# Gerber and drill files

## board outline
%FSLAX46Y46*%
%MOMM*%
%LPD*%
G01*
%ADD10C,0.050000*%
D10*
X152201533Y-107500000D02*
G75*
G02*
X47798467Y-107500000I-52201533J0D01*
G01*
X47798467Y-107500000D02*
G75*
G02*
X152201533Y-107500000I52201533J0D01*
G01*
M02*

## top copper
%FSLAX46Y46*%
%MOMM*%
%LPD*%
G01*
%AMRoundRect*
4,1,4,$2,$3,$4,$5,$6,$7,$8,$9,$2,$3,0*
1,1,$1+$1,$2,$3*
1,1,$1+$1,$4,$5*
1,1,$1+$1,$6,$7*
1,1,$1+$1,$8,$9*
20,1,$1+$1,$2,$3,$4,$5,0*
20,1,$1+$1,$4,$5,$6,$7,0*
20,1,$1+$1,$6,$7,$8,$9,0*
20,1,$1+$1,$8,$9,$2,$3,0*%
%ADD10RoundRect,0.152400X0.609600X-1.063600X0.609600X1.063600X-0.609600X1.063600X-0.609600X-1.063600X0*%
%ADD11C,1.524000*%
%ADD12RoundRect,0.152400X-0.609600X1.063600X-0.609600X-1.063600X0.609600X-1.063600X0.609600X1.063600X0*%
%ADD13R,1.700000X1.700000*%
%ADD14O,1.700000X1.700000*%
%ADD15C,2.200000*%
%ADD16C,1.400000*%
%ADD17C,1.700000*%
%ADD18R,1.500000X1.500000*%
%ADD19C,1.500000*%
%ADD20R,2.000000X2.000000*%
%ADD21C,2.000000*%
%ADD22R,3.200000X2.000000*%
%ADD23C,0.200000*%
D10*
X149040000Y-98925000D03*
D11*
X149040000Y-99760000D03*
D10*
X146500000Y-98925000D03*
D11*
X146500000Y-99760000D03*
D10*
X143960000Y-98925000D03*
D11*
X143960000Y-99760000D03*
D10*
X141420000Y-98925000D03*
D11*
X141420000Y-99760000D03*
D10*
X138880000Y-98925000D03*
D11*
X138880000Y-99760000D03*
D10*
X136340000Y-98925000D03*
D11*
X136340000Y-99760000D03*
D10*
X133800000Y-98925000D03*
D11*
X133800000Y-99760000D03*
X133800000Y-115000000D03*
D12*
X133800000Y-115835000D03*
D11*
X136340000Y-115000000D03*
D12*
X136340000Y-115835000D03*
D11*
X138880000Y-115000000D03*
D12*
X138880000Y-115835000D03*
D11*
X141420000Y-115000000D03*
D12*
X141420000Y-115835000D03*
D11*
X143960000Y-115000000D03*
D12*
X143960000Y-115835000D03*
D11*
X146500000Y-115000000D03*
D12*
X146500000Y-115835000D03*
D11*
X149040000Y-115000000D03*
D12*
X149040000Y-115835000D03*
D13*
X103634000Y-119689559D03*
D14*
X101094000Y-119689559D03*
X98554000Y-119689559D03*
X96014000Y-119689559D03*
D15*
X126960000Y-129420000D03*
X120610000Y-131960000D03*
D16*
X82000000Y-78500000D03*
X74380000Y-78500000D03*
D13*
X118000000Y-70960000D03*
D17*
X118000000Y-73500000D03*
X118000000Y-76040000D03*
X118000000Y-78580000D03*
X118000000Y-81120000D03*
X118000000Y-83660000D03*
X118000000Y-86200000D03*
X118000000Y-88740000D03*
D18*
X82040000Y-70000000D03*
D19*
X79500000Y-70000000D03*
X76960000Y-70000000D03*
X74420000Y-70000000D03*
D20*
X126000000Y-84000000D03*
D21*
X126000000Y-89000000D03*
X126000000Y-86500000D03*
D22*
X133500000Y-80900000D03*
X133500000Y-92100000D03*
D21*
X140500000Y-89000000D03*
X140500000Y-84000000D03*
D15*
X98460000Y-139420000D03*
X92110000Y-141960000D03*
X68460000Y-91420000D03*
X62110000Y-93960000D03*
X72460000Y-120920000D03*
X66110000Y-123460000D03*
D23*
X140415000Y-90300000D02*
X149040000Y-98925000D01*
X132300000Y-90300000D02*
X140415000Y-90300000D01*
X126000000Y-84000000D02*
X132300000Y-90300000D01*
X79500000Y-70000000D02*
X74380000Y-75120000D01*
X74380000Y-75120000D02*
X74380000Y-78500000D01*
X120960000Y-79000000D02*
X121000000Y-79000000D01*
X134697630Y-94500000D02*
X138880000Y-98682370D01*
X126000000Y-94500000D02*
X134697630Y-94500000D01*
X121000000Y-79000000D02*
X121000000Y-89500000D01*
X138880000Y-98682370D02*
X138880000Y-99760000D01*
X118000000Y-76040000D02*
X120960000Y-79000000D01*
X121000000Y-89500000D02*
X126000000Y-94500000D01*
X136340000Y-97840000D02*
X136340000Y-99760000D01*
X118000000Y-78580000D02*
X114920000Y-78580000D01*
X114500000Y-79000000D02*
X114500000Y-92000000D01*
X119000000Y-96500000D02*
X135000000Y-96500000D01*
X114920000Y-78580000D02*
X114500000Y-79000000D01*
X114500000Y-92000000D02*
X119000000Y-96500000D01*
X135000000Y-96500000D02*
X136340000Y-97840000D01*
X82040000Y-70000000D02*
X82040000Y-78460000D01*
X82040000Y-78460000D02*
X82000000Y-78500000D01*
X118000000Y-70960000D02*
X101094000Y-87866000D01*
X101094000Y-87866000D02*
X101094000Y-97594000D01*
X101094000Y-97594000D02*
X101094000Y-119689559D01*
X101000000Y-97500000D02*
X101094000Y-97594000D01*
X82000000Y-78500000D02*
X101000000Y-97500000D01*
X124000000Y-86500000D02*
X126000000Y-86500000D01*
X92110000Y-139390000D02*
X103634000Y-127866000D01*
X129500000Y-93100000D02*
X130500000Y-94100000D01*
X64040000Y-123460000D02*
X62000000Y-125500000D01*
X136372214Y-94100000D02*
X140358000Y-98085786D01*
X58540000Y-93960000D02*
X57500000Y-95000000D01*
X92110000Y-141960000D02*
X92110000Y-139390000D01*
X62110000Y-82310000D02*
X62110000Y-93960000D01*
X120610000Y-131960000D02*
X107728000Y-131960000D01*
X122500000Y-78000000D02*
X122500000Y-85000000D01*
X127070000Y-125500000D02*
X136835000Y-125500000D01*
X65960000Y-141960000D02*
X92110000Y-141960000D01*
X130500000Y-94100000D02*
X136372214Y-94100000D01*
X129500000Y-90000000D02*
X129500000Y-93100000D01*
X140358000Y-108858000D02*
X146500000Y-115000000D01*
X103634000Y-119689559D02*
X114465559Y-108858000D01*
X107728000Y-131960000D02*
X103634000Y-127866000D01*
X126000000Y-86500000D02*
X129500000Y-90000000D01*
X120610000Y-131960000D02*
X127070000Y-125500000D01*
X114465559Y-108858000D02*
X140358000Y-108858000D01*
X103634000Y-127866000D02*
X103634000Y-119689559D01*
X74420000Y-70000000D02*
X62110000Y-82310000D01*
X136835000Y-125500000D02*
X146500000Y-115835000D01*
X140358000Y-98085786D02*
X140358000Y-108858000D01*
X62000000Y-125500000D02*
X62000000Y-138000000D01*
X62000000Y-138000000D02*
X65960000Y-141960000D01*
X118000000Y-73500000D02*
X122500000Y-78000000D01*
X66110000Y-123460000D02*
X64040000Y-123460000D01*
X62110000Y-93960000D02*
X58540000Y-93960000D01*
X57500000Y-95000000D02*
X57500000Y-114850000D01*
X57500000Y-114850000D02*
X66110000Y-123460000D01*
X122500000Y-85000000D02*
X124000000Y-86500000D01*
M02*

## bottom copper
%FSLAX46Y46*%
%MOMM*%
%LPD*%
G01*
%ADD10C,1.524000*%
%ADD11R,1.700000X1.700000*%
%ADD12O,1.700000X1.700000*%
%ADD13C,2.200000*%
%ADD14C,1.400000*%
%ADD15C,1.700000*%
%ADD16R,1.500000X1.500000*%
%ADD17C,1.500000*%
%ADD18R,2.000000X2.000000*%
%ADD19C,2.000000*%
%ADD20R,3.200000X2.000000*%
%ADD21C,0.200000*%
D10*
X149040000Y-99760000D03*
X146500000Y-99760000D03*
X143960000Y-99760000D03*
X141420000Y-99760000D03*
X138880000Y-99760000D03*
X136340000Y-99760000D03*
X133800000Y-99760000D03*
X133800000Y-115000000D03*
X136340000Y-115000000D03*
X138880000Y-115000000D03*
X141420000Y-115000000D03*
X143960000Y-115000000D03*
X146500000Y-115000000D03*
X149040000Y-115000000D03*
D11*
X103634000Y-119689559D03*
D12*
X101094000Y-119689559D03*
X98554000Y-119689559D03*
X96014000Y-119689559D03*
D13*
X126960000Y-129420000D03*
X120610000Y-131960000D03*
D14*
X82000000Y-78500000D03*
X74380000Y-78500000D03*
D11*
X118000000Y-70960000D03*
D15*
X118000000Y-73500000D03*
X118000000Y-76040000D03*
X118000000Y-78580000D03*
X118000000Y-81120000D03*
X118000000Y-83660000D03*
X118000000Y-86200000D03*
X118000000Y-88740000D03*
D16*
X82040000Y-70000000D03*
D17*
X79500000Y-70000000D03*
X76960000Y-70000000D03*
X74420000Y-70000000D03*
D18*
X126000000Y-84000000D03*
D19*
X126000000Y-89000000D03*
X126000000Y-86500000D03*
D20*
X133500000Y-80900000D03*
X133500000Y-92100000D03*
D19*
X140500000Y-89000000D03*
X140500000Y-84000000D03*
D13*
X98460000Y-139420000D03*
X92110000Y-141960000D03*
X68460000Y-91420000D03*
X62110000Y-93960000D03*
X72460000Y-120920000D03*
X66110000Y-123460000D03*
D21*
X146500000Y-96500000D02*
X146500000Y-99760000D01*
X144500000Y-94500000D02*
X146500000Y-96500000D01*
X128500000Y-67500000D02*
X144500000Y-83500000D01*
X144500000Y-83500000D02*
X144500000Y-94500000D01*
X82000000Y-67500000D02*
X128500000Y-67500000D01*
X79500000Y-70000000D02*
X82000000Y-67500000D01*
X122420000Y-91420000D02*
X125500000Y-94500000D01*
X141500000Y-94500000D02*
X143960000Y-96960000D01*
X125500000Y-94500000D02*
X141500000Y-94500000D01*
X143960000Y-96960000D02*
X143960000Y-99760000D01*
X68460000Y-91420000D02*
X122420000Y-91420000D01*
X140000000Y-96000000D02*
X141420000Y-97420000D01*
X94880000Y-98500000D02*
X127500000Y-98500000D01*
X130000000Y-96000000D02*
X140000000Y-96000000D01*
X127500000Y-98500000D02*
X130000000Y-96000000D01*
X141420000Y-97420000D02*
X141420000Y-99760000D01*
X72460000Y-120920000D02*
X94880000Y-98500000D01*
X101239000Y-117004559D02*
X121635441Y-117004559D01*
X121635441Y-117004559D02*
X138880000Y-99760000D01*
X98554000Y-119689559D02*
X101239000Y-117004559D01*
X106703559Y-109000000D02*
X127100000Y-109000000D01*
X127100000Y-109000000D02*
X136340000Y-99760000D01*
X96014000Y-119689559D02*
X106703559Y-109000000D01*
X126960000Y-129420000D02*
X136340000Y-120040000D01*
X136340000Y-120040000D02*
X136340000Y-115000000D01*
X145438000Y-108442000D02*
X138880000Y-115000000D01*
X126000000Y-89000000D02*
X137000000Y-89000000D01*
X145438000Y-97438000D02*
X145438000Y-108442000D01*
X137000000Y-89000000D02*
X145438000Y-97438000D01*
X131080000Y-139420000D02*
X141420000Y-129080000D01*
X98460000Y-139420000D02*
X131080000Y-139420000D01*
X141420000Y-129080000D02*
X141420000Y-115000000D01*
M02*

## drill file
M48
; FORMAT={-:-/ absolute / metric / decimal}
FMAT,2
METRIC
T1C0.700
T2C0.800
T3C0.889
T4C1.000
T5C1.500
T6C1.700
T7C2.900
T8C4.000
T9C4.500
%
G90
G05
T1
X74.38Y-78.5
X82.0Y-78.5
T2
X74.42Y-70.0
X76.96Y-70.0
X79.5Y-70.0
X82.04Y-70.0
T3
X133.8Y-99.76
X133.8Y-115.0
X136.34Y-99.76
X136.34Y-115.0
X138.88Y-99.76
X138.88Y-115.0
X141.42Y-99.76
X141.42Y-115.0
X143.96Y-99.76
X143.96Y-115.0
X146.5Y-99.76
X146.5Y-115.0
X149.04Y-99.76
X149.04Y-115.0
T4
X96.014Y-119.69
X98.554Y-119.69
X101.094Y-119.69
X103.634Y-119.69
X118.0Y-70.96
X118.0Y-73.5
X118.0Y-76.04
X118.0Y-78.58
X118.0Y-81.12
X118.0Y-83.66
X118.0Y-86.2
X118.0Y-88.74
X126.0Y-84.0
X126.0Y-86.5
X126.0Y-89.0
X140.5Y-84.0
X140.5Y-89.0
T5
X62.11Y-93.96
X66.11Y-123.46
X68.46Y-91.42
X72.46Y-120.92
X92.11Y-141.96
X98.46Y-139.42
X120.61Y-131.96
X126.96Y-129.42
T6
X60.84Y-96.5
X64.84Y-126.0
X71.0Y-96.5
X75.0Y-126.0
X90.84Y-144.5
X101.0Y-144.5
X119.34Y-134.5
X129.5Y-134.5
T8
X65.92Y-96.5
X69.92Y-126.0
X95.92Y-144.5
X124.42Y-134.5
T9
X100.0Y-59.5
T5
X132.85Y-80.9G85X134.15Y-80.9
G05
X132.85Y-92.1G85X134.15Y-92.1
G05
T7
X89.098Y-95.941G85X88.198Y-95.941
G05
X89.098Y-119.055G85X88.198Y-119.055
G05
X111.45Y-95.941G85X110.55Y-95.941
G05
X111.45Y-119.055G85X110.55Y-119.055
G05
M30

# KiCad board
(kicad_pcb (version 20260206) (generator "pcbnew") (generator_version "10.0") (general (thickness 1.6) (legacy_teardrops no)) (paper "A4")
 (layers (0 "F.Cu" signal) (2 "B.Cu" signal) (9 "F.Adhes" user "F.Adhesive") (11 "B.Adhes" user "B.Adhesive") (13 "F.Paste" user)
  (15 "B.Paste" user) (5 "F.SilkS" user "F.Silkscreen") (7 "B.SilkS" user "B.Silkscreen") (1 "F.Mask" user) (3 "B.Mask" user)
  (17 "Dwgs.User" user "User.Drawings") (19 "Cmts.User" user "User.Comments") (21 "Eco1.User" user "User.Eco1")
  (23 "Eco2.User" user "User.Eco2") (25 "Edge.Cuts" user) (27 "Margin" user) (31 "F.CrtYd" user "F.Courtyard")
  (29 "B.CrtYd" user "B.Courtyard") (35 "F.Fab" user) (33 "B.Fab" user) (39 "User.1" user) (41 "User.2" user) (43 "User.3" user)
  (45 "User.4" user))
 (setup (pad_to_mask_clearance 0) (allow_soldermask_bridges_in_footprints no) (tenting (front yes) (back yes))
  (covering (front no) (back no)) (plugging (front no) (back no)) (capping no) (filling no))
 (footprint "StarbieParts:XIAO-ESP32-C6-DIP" (layer "F.Cu") (at 141.42 107.38)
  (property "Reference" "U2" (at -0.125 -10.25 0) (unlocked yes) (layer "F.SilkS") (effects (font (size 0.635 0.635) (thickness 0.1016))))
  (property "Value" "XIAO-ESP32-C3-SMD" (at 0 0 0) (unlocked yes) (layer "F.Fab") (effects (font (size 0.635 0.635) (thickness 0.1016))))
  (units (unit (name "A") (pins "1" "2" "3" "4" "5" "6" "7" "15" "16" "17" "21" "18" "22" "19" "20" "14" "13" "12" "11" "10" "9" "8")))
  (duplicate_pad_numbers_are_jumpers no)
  (pad "1" smd roundrect (at 7.62 -8.455 90) (size 2.432 1.524) (layers "F.Cu" "F.Mask") (roundrect_rratio 0.1) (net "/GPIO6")
   (thermal_bridge_angle 45))
  (pad "1" thru_hole circle (at 7.62 -7.62 90) (size 1.524 1.524) (drill 0.889) (layers "*.Cu" "*.Mask") (remove_unused_layers no)
   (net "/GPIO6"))
  (pad "2" smd roundrect (at 5.08 -8.455 90) (size 2.432 1.524) (layers "F.Cu" "F.Mask") (roundrect_rratio 0.1) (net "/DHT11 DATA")
   (thermal_bridge_angle 45))
  (pad "2" thru_hole circle (at 5.08 -7.62 90) (size 1.524 1.524) (drill 0.889) (layers "*.Cu" "*.Mask") (remove_unused_layers no)
   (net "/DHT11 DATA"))
  (pad "3" smd roundrect (at 2.54 -8.455 90) (size 2.432 1.524) (layers "F.Cu" "F.Mask") (roundrect_rratio 0.1) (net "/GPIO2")
   (thermal_bridge_angle 45))
  (pad "3" thru_hole circle (at 2.54 -7.62 90) (size 1.524 1.524) (drill 0.889) (layers "*.Cu" "*.Mask") (remove_unused_layers no)
   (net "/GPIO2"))
  (pad "4" smd roundrect (at 0 -8.455 90) (size 2.432 1.524) (layers "F.Cu" "F.Mask") (roundrect_rratio 0.1) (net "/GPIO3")
   (thermal_bridge_angle 45))
  (pad "4" thru_hole circle (at 0 -7.62 90) (size 1.524 1.524) (drill 0.889) (layers "*.Cu" "*.Mask") (remove_unused_layers no)
   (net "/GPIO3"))
  (pad "5" smd roundrect (at -2.54 -8.455 90) (size 2.432 1.524) (layers "F.Cu" "F.Mask") (roundrect_rratio 0.1) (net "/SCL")
   (thermal_bridge_angle 45))
  (pad "5" thru_hole circle (at -2.54 -7.62 90) (size 1.524 1.524) (drill 0.889) (layers "*.Cu" "*.Mask") (remove_unused_layers no)
   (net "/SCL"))
  (pad "6" smd roundrect (at -5.08 -8.455 90) (size 2.432 1.524) (layers "F.Cu" "F.Mask") (roundrect_rratio 0.1) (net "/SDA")
   (thermal_bridge_angle 45))
  (pad "6" thru_hole circle (at -5.08 -7.62 90) (size 1.524 1.524) (drill 0.889) (layers "*.Cu" "*.Mask") (remove_unused_layers no)
   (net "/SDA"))
  (pad "7" smd roundrect (at -7.62 -8.455 90) (size 2.432 1.524) (layers "F.Cu" "F.Mask") (roundrect_rratio 0.1)
   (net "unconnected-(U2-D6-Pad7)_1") (thermal_bridge_angle 45))
  (pad "7" thru_hole circle (at -7.62 -7.62 90) (size 1.524 1.524) (drill 0.889) (layers "*.Cu" "*.Mask") (remove_unused_layers no)
   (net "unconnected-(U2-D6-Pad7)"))
  (pad "8" thru_hole circle (at -7.62 7.62 270) (size 1.524 1.524) (drill 0.889) (layers "*.Cu" "*.Mask") (remove_unused_layers no)
   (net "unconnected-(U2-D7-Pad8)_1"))
  (pad "8" smd roundrect (at -7.62 8.455 270) (size 2.432 1.524) (layers "F.Cu" "F.Mask") (roundrect_rratio 0.1)
   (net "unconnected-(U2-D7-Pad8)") (thermal_bridge_angle 45))
  (pad "9" thru_hole circle (at -5.08 7.62 270) (size 1.524 1.524) (drill 0.889) (layers "*.Cu" "*.Mask") (remove_unused_layers no)
   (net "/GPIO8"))
  (pad "9" smd roundrect (at -5.08 8.455 270) (size 2.432 1.524) (layers "F.Cu" "F.Mask") (roundrect_rratio 0.1) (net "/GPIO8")
   (thermal_bridge_angle 45))
  (pad "10" thru_hole circle (at -2.54 7.62 270) (size 1.524 1.524) (drill 0.889) (layers "*.Cu" "*.Mask") (remove_unused_layers no)
   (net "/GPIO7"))
  (pad "10" smd roundrect (at -2.54 8.455 270) (size 2.432 1.524) (layers "F.Cu" "F.Mask") (roundrect_rratio 0.1) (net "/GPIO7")
   (thermal_bridge_angle 45))
  (pad "11" thru_hole circle (at 0 7.62 270) (size 1.524 1.524) (drill 0.889) (layers "*.Cu" "*.Mask") (remove_unused_layers no)
   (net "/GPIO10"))
  (pad "11" smd roundrect (at 0 8.455 270) (size 2.432 1.524) (layers "F.Cu" "F.Mask") (roundrect_rratio 0.1) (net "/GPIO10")
   (thermal_bridge_angle 45))
  (pad "12" thru_hole circle (at 2.54 7.62 270) (size 1.524 1.524) (drill 0.889) (layers "*.Cu" "*.Mask") (remove_unused_layers no)
   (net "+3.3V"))
  (pad "12" smd roundrect (at 2.54 8.455 270) (size 2.432 1.524) (layers "F.Cu" "F.Mask") (roundrect_rratio 0.1) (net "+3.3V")
   (thermal_bridge_angle 45))
  (pad "13" thru_hole circle (at 5.08 7.62 270) (size 1.524 1.524) (drill 0.889) (layers "*.Cu" "*.Mask") (remove_unused_layers no)
   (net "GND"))
  (pad "13" smd roundrect (at 5.08 8.455 270) (size 2.432 1.524) (layers "F.Cu" "F.Mask") (roundrect_rratio 0.1) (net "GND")
   (thermal_bridge_angle 45))
  (pad "14" thru_hole circle (at 7.62 7.62 270) (size 1.524 1.524) (drill 0.889) (layers "*.Cu" "*.Mask") (remove_unused_layers no)
   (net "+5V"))
  (pad "14" smd roundrect (at 7.62 8.455 270) (size 2.432 1.524) (layers "F.Cu" "F.Mask") (roundrect_rratio 0.1) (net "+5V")
   (thermal_bridge_angle 45)))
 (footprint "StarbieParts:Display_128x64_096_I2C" (layer "F.Cu") (at 99.824 119.689559 180)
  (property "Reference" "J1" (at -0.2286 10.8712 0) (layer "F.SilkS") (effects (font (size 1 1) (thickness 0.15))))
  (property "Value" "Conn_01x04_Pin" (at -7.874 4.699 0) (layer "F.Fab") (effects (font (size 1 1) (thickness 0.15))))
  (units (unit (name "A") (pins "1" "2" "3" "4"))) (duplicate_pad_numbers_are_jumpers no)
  (pad "" np_thru_hole oval (at -11.176 0.635 180) (size 3.8 2.9) (drill oval 3.8 2.9) (layers "*.Cu" "*.Mask"))
  (pad "" np_thru_hole oval (at -11.176 23.749 180) (size 3.8 2.9) (drill oval 3.8 2.9) (layers "*.Cu" "*.Mask"))
  (pad "" np_thru_hole oval (at 11.176 0.635 180) (size 3.8 2.9) (drill oval 3.8 2.9) (layers "*.Cu" "*.Mask"))
  (pad "" np_thru_hole oval (at 11.176 23.749 180) (size 3.8 2.9) (drill oval 3.8 2.9) (layers "*.Cu" "*.Mask"))
  (pad "1" thru_hole rect (at -3.81 0 270) (size 1.7 1.7) (drill 1) (layers "*.Cu" "*.Mask") (remove_unused_layers no) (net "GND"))
  (pad "2" thru_hole oval (at -1.27 0 270) (size 1.7 1.7) (drill 1) (layers "*.Cu" "*.Mask") (remove_unused_layers no) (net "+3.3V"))
  (pad "3" thru_hole oval (at 1.27 0 270) (size 1.7 1.7) (drill 1) (layers "*.Cu" "*.Mask") (remove_unused_layers no) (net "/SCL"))
  (pad "4" thru_hole oval (at 3.81 0 270) (size 1.7 1.7) (drill 1) (layers "*.Cu" "*.Mask") (remove_unused_layers no) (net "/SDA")))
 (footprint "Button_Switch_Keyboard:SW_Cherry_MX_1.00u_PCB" (layer "F.Cu") (at 126.96 129.42)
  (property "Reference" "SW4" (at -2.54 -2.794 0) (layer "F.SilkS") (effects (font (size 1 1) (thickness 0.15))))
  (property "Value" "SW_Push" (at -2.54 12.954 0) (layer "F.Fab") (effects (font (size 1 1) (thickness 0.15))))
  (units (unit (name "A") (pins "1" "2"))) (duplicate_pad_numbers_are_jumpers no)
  (pad "" np_thru_hole circle (at -7.62 5.08) (size 1.7 1.7) (drill 1.7) (layers "*.Cu" "*.Mask"))
  (pad "" np_thru_hole circle (at -2.54 5.08) (size 4 4) (drill 4) (layers "*.Cu" "*.Mask"))
  (pad "" np_thru_hole circle (at 2.54 5.08) (size 1.7 1.7) (drill 1.7) (layers "*.Cu" "*.Mask"))
  (pad "1" thru_hole circle (at 0 0) (size 2.2 2.2) (drill 1.5) (layers "*.Cu" "*.Mask") (remove_unused_layers no) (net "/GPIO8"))
  (pad "2" thru_hole circle (at -6.35 2.54) (size 2.2 2.2) (drill 1.5) (layers "*.Cu" "*.Mask") (remove_unused_layers no) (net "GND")))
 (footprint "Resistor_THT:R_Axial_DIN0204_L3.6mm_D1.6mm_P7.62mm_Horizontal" (layer "F.Cu") (at 82 78.5 180)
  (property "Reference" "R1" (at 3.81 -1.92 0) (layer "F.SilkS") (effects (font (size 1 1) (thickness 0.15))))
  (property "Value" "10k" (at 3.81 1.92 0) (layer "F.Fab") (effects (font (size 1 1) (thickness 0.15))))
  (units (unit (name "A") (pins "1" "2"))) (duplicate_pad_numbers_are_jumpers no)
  (pad "1" thru_hole circle (at 0 0 180) (size 1.4 1.4) (drill 0.7) (layers "*.Cu" "*.Mask") (remove_unused_layers no) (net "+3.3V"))
  (pad "2" thru_hole circle (at 7.62 0 180) (size 1.4 1.4) (drill 0.7) (layers "*.Cu" "*.Mask") (remove_unused_layers no)
   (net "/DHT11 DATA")))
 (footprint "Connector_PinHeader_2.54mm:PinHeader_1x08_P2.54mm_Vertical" (layer "F.Cu") (at 118 70.96)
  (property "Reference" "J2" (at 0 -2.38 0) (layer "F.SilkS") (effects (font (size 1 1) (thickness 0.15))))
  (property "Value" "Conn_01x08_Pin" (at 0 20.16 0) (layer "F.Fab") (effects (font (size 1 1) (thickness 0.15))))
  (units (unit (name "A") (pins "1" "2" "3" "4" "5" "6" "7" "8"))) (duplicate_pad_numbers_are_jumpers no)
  (pad "1" thru_hole rect (at 0 0) (size 1.7 1.7) (drill 1) (layers "*.Cu" "*.Mask") (remove_unused_layers no) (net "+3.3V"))
  (pad "2" thru_hole circle (at 0 2.54) (size 1.7 1.7) (drill 1) (layers "*.Cu" "*.Mask") (remove_unused_layers no) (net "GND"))
  (pad "3" thru_hole circle (at 0 5.08) (size 1.7 1.7) (drill 1) (layers "*.Cu" "*.Mask") (remove_unused_layers no) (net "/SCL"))
  (pad "4" thru_hole circle (at 0 7.62) (size 1.7 1.7) (drill 1) (layers "*.Cu" "*.Mask") (remove_unused_layers no) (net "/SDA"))
  (pad "5" thru_hole circle (at 0 10.16) (size 1.7 1.7) (drill 1) (layers "*.Cu" "*.Mask") (remove_unused_layers no)
   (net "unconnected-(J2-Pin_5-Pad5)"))
  (pad "6" thru_hole circle (at 0 12.7) (size 1.7 1.7) (drill 1) (layers "*.Cu" "*.Mask") (remove_unused_layers no)
   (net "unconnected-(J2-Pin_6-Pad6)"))
  (pad "7" thru_hole circle (at 0 15.24) (size 1.7 1.7) (drill 1) (layers "*.Cu" "*.Mask") (remove_unused_layers no)
   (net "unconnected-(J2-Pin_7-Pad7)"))
  (pad "8" thru_hole circle (at 0 17.78) (size 1.7 1.7) (drill 1) (layers "*.Cu" "*.Mask") (remove_unused_layers no)
   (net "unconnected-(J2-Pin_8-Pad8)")))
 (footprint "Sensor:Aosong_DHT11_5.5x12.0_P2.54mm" (layer "F.Cu") (at 82.04 70 -90)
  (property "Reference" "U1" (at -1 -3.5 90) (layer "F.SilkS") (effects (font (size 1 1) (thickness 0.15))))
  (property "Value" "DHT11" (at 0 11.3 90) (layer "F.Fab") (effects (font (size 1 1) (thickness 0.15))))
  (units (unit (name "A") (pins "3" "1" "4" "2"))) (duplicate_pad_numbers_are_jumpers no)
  (pad "1" thru_hole rect (at 0 0 270) (size 1.5 1.5) (drill 0.8) (layers "*.Cu" "*.Mask") (remove_unused_layers no) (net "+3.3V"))
  (pad "2" thru_hole circle (at 0 2.54 270) (size 1.5 1.5) (drill 0.8) (layers "*.Cu" "*.Mask") (remove_unused_layers no)
   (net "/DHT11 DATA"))
  (pad "3" thru_hole circle (at 0 5.08 270) (size 1.5 1.5) (drill 0.8) (layers "*.Cu" "*.Mask") (remove_unused_layers no)
   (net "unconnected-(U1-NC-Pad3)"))
  (pad "4" thru_hole circle (at 0 7.62 270) (size 1.5 1.5) (drill 0.8) (layers "*.Cu" "*.Mask") (remove_unused_layers no) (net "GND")))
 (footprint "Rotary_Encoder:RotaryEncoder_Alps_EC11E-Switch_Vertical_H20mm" (layer "F.Cu") (at 126 84)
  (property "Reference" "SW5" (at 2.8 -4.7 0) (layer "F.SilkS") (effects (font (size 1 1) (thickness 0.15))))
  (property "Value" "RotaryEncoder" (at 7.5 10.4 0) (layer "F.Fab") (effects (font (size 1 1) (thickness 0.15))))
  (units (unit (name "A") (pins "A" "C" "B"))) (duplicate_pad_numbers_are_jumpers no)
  (pad "A" thru_hole rect (at 0 0) (size 2 2) (drill 1) (layers "*.Cu" "*.Mask") (remove_unused_layers no) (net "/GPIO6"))
  (pad "B" thru_hole circle (at 0 5) (size 2 2) (drill 1) (layers "*.Cu" "*.Mask") (remove_unused_layers no) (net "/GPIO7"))
  (pad "C" thru_hole circle (at 0 2.5) (size 2 2) (drill 1) (layers "*.Cu" "*.Mask") (remove_unused_layers no) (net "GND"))
  (pad "MP" thru_hole rect (at 7.5 -3.1) (size 3.2 2) (drill oval 2.8 1.5) (layers "*.Cu" "*.Mask") (remove_unused_layers no))
  (pad "MP" thru_hole rect (at 7.5 8.1) (size 3.2 2) (drill oval 2.8 1.5) (layers "*.Cu" "*.Mask") (remove_unused_layers no))
  (pad "S1" thru_hole circle (at 14.5 5) (size 2 2) (drill 1) (layers "*.Cu" "*.Mask") (remove_unused_layers no))
  (pad "S2" thru_hole circle (at 14.5 0) (size 2 2) (drill 1) (layers "*.Cu" "*.Mask") (remove_unused_layers no)))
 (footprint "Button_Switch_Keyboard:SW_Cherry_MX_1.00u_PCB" (layer "F.Cu") (at 98.46 139.42)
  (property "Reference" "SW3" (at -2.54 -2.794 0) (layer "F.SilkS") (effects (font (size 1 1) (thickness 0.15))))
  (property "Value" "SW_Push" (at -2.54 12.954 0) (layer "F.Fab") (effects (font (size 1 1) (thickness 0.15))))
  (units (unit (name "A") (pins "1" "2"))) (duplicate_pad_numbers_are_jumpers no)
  (pad "" np_thru_hole circle (at -7.62 5.08) (size 1.7 1.7) (drill 1.7) (layers "*.Cu" "*.Mask"))
  (pad "" np_thru_hole circle (at -2.54 5.08) (size 4 4) (drill 4) (layers "*.Cu" "*.Mask"))
  (pad "" np_thru_hole circle (at 2.54 5.08) (size 1.7 1.7) (drill 1.7) (layers "*.Cu" "*.Mask"))
  (pad "1" thru_hole circle (at 0 0) (size 2.2 2.2) (drill 1.5) (layers "*.Cu" "*.Mask") (remove_unused_layers no) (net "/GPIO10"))
  (pad "2" thru_hole circle (at -6.35 2.54) (size 2.2 2.2) (drill 1.5) (layers "*.Cu" "*.Mask") (remove_unused_layers no) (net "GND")))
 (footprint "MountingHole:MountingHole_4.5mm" (layer "F.Cu") (at 100 59.5)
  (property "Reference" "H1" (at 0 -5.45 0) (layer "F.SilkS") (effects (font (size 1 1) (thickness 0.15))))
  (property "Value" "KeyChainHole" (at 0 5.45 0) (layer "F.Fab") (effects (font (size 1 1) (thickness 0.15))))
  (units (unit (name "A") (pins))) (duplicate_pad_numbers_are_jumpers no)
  (pad "" np_thru_hole circle (at 0 0) (size 4.5 4.5) (drill 4.5) (layers "*.Cu" "*.Mask")))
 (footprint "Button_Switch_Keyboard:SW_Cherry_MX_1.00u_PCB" (layer "F.Cu") (at 68.46 91.42)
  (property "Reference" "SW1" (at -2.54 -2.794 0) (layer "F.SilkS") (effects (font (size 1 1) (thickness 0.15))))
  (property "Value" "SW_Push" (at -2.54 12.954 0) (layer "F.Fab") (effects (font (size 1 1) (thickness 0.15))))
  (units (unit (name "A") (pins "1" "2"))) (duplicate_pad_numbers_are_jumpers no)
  (pad "" np_thru_hole circle (at -7.62 5.08) (size 1.7 1.7) (drill 1.7) (layers "*.Cu" "*.Mask"))
  (pad "" np_thru_hole circle (at -2.54 5.08) (size 4 4) (drill 4) (layers "*.Cu" "*.Mask"))
  (pad "" np_thru_hole circle (at 2.54 5.08) (size 1.7 1.7) (drill 1.7) (layers "*.Cu" "*.Mask"))
  (pad "1" thru_hole circle (at 0 0) (size 2.2 2.2) (drill 1.5) (layers "*.Cu" "*.Mask") (remove_unused_layers no) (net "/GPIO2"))
  (pad "2" thru_hole circle (at -6.35 2.54) (size 2.2 2.2) (drill 1.5) (layers "*.Cu" "*.Mask") (remove_unused_layers no) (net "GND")))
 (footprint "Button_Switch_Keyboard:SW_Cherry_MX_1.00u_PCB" (layer "F.Cu") (at 72.46 120.92)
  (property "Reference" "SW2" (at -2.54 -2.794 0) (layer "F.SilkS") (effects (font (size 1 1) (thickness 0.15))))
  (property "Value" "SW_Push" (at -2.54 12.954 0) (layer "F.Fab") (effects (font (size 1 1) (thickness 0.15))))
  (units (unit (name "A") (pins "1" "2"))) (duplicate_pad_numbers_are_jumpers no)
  (pad "" np_thru_hole circle (at -7.62 5.08) (size 1.7 1.7) (drill 1.7) (layers "*.Cu" "*.Mask"))
  (pad "" np_thru_hole circle (at -2.54 5.08) (size 4 4) (drill 4) (layers "*.Cu" "*.Mask"))
  (pad "" np_thru_hole circle (at 2.54 5.08) (size 1.7 1.7) (drill 1.7) (layers "*.Cu" "*.Mask"))
  (pad "1" thru_hole circle (at 0 0) (size 2.2 2.2) (drill 1.5) (layers "*.Cu" "*.Mask") (remove_unused_layers no) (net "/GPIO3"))
  (pad "2" thru_hole circle (at -6.35 2.54) (size 2.2 2.2) (drill 1.5) (layers "*.Cu" "*.Mask") (remove_unused_layers no) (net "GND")))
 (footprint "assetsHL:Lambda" (layer "F.Cu") (at 99.824 107.681559)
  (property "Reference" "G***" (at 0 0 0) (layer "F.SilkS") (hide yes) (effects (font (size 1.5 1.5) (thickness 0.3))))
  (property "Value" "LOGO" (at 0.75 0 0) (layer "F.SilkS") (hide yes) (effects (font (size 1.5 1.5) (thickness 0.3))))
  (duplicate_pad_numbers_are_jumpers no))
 (gr_circle (center 100 107.5) (end 149 125.5) (stroke (width 0.05) (type default)) (fill no) (layer "Edge.Cuts"))
 (segment (start 140.415 90.3) (end 149.04 98.925) (width 0.2) (layer "F.Cu") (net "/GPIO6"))
 (segment (start 132.3 90.3) (end 140.415 90.3) (width 0.2) (layer "F.Cu") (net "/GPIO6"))
 (segment (start 126 84) (end 132.3 90.3) (width 0.2) (layer "F.Cu") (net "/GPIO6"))
 (segment (start 79.5 70) (end 74.38 75.12) (width 0.2) (layer "F.Cu") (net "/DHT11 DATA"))
 (segment (start 74.38 75.12) (end 74.38 78.5) (width 0.2) (layer "F.Cu") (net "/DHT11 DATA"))
 (segment (start 146.5 96.5) (end 146.5 99.76) (width 0.2) (layer "B.Cu") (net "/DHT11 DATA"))
 (segment (start 144.5 94.5) (end 146.5 96.5) (width 0.2) (layer "B.Cu") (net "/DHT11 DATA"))
 (segment (start 128.5 67.5) (end 144.5 83.5) (width 0.2) (layer "B.Cu") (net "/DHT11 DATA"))
 (segment (start 144.5 83.5) (end 144.5 94.5) (width 0.2) (layer "B.Cu") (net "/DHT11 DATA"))
 (segment (start 82 67.5) (end 128.5 67.5) (width 0.2) (layer "B.Cu") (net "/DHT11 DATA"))
 (segment (start 79.5 70) (end 82 67.5) (width 0.2) (layer "B.Cu") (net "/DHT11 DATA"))
 (segment (start 122.42 91.42) (end 125.5 94.5) (width 0.2) (layer "B.Cu") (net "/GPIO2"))
 (segment (start 141.5 94.5) (end 143.96 96.96) (width 0.2) (layer "B.Cu") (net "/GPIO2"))
 (segment (start 125.5 94.5) (end 141.5 94.5) (width 0.2) (layer "B.Cu") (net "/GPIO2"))
 (segment (start 143.96 96.96) (end 143.96 99.76) (width 0.2) (layer "B.Cu") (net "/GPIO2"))
 (segment (start 68.46 91.42) (end 122.42 91.42) (width 0.2) (layer "B.Cu") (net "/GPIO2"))
 (segment (start 140 96) (end 141.42 97.42) (width 0.2) (layer "B.Cu") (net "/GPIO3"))
 (segment (start 94.88 98.5) (end 127.5 98.5) (width 0.2) (layer "B.Cu") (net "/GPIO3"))
 (segment (start 130 96) (end 140 96) (width 0.2) (layer "B.Cu") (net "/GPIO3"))
 (segment (start 127.5 98.5) (end 130 96) (width 0.2) (layer "B.Cu") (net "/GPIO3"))
 (segment (start 141.42 97.42) (end 141.42 99.76) (width 0.2) (layer "B.Cu") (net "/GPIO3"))
 (segment (start 72.46 120.92) (end 94.88 98.5) (width 0.2) (layer "B.Cu") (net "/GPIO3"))
 (segment (start 120.96 79) (end 121 79) (width 0.2) (layer "F.Cu") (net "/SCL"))
 (segment (start 134.69763 94.5) (end 138.88 98.68237) (width 0.2) (layer "F.Cu") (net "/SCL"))
 (segment (start 126 94.5) (end 134.69763 94.5) (width 0.2) (layer "F.Cu") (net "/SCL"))
 (segment (start 121 79) (end 121 89.5) (width 0.2) (layer "F.Cu") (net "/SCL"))
 (segment (start 138.88 98.68237) (end 138.88 99.76) (width 0.2) (layer "F.Cu") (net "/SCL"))
 (segment (start 118 76.04) (end 120.96 79) (width 0.2) (layer "F.Cu") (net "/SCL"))
 (segment (start 121 89.5) (end 126 94.5) (width 0.2) (layer "F.Cu") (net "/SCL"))
 (segment (start 101.239 117.004559) (end 121.635441 117.004559) (width 0.2) (layer "B.Cu") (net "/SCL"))
 (segment (start 121.635441 117.004559) (end 138.88 99.76) (width 0.2) (layer "B.Cu") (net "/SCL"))
 (segment (start 98.554 119.689559) (end 101.239 117.004559) (width 0.2) (layer "B.Cu") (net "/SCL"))
 (segment (start 136.34 97.84) (end 136.34 99.76) (width 0.2) (layer "F.Cu") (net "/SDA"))
 (segment (start 118 78.58) (end 114.92 78.58) (width 0.2) (layer "F.Cu") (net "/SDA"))
 (segment (start 114.5 79) (end 114.5 92) (width 0.2) (layer "F.Cu") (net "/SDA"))
 (segment (start 119 96.5) (end 135 96.5) (width 0.2) (layer "F.Cu") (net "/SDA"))
 (segment (start 114.92 78.58) (end 114.5 79) (width 0.2) (layer "F.Cu") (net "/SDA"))
 (segment (start 114.5 92) (end 119 96.5) (width 0.2) (layer "F.Cu") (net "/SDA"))
 (segment (start 135 96.5) (end 136.34 97.84) (width 0.2) (layer "F.Cu") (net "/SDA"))
 (segment (start 106.703559 109) (end 127.1 109) (width 0.2) (layer "B.Cu") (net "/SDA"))
 (segment (start 127.1 109) (end 136.34 99.76) (width 0.2) (layer "B.Cu") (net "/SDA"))
 (segment (start 96.014 119.689559) (end 106.703559 109) (width 0.2) (layer "B.Cu") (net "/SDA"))
 (segment (start 126.96 129.42) (end 136.34 120.04) (width 0.2) (layer "B.Cu") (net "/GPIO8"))
 (segment (start 136.34 120.04) (end 136.34 115) (width 0.2) (layer "B.Cu") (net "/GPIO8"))
 (segment (start 145.438 108.442) (end 138.88 115) (width 0.2) (layer "B.Cu") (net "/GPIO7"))
 (segment (start 126 89) (end 137 89) (width 0.2) (layer "B.Cu") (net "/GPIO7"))
 (segment (start 145.438 97.438) (end 145.438 108.442) (width 0.2) (layer "B.Cu") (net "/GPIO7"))
 (segment (start 137 89) (end 145.438 97.438) (width 0.2) (layer "B.Cu") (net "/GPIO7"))
 (segment (start 131.08 139.42) (end 141.42 129.08) (width 0.2) (layer "B.Cu") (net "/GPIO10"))
 (segment (start 98.46 139.42) (end 131.08 139.42) (width 0.2) (layer "B.Cu") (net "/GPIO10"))
 (segment (start 141.42 129.08) (end 141.42 115) (width 0.2) (layer "B.Cu") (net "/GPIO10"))
 (segment (start 82.04 70) (end 82.04 78.46) (width 0.2) (layer "F.Cu") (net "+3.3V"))
 (segment (start 82.04 78.46) (end 82 78.5) (width 0.2) (layer "F.Cu") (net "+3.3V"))
 (segment (start 118 70.96) (end 101.094 87.866) (width 0.2) (layer "F.Cu") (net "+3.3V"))
 (segment (start 101.094 87.866) (end 101.094 97.594) (width 0.2) (layer "F.Cu") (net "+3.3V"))
 (segment (start 101.094 97.594) (end 101.094 119.689559) (width 0.2) (layer "F.Cu") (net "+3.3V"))
 (segment (start 101 97.5) (end 101.094 97.594) (width 0.2) (layer "F.Cu") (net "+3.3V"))
 (segment (start 82 78.5) (end 101 97.5) (width 0.2) (layer "F.Cu") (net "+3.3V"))
 (segment (start 124 86.5) (end 126 86.5) (width 0.2) (layer "F.Cu") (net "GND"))
 (segment (start 92.11 139.39) (end 103.634 127.866) (width 0.2) (layer "F.Cu") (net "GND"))
 (segment (start 129.5 93.1) (end 130.5 94.1) (width 0.2) (layer "F.Cu") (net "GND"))
 (segment (start 64.04 123.46) (end 62 125.5) (width 0.2) (layer "F.Cu") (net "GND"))
 (segment (start 136.372214 94.1) (end 140.358 98.085786) (width 0.2) (layer "F.Cu") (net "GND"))
 (segment (start 58.54 93.96) (end 57.5 95) (width 0.2) (layer "F.Cu") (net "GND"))
 (segment (start 92.11 141.96) (end 92.11 139.39) (width 0.2) (layer "F.Cu") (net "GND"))
 (segment (start 62.11 82.31) (end 62.11 93.96) (width 0.2) (layer "F.Cu") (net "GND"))
 (segment (start 120.61 131.96) (end 107.728 131.96) (width 0.2) (layer "F.Cu") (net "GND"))
 (segment (start 122.5 78) (end 122.5 85) (width 0.2) (layer "F.Cu") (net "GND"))
 (segment (start 127.07 125.5) (end 136.835 125.5) (width 0.2) (layer "F.Cu") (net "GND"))
 (segment (start 65.96 141.96) (end 92.11 141.96) (width 0.2) (layer "F.Cu") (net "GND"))
 (segment (start 130.5 94.1) (end 136.372214 94.1) (width 0.2) (layer "F.Cu") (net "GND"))
 (segment (start 129.5 90) (end 129.5 93.1) (width 0.2) (layer "F.Cu") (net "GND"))
 (segment (start 140.358 108.858) (end 146.5 115) (width 0.2) (layer "F.Cu") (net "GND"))
 (segment (start 103.634 119.689559) (end 114.465559 108.858) (width 0.2) (layer "F.Cu") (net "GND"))
 (segment (start 107.728 131.96) (end 103.634 127.866) (width 0.2) (layer "F.Cu") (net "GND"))
 (segment (start 126 86.5) (end 129.5 90) (width 0.2) (layer "F.Cu") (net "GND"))
 (segment (start 120.61 131.96) (end 127.07 125.5) (width 0.2) (layer "F.Cu") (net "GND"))
 (segment (start 114.465559 108.858) (end 140.358 108.858) (width 0.2) (layer "F.Cu") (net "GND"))
 (segment (start 103.634 127.866) (end 103.634 119.689559) (width 0.2) (layer "F.Cu") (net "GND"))
 (segment (start 74.42 70) (end 62.11 82.31) (width 0.2) (layer "F.Cu") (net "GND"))
 (segment (start 136.835 125.5) (end 146.5 115.835) (width 0.2) (layer "F.Cu") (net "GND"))
 (segment (start 140.358 98.085786) (end 140.358 108.858) (width 0.2) (layer "F.Cu") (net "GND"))
 (segment (start 62 125.5) (end 62 138) (width 0.2) (layer "F.Cu") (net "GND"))
 (segment (start 62 138) (end 65.96 141.96) (width 0.2) (layer "F.Cu") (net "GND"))
 (segment (start 118 73.5) (end 122.5 78) (width 0.2) (layer "F.Cu") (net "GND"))
 (segment (start 66.11 123.46) (end 64.04 123.46) (width 0.2) (layer "F.Cu") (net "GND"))
 (segment (start 62.11 93.96) (end 58.54 93.96) (width 0.2) (layer "F.Cu") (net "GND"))
 (segment (start 57.5 95) (end 57.5 114.85) (width 0.2) (layer "F.Cu") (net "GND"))
 (segment (start 57.5 114.85) (end 66.11 123.46) (width 0.2) (layer "F.Cu") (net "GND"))
 (segment (start 122.5 85) (end 124 86.5) (width 0.2) (layer "F.Cu") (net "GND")))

